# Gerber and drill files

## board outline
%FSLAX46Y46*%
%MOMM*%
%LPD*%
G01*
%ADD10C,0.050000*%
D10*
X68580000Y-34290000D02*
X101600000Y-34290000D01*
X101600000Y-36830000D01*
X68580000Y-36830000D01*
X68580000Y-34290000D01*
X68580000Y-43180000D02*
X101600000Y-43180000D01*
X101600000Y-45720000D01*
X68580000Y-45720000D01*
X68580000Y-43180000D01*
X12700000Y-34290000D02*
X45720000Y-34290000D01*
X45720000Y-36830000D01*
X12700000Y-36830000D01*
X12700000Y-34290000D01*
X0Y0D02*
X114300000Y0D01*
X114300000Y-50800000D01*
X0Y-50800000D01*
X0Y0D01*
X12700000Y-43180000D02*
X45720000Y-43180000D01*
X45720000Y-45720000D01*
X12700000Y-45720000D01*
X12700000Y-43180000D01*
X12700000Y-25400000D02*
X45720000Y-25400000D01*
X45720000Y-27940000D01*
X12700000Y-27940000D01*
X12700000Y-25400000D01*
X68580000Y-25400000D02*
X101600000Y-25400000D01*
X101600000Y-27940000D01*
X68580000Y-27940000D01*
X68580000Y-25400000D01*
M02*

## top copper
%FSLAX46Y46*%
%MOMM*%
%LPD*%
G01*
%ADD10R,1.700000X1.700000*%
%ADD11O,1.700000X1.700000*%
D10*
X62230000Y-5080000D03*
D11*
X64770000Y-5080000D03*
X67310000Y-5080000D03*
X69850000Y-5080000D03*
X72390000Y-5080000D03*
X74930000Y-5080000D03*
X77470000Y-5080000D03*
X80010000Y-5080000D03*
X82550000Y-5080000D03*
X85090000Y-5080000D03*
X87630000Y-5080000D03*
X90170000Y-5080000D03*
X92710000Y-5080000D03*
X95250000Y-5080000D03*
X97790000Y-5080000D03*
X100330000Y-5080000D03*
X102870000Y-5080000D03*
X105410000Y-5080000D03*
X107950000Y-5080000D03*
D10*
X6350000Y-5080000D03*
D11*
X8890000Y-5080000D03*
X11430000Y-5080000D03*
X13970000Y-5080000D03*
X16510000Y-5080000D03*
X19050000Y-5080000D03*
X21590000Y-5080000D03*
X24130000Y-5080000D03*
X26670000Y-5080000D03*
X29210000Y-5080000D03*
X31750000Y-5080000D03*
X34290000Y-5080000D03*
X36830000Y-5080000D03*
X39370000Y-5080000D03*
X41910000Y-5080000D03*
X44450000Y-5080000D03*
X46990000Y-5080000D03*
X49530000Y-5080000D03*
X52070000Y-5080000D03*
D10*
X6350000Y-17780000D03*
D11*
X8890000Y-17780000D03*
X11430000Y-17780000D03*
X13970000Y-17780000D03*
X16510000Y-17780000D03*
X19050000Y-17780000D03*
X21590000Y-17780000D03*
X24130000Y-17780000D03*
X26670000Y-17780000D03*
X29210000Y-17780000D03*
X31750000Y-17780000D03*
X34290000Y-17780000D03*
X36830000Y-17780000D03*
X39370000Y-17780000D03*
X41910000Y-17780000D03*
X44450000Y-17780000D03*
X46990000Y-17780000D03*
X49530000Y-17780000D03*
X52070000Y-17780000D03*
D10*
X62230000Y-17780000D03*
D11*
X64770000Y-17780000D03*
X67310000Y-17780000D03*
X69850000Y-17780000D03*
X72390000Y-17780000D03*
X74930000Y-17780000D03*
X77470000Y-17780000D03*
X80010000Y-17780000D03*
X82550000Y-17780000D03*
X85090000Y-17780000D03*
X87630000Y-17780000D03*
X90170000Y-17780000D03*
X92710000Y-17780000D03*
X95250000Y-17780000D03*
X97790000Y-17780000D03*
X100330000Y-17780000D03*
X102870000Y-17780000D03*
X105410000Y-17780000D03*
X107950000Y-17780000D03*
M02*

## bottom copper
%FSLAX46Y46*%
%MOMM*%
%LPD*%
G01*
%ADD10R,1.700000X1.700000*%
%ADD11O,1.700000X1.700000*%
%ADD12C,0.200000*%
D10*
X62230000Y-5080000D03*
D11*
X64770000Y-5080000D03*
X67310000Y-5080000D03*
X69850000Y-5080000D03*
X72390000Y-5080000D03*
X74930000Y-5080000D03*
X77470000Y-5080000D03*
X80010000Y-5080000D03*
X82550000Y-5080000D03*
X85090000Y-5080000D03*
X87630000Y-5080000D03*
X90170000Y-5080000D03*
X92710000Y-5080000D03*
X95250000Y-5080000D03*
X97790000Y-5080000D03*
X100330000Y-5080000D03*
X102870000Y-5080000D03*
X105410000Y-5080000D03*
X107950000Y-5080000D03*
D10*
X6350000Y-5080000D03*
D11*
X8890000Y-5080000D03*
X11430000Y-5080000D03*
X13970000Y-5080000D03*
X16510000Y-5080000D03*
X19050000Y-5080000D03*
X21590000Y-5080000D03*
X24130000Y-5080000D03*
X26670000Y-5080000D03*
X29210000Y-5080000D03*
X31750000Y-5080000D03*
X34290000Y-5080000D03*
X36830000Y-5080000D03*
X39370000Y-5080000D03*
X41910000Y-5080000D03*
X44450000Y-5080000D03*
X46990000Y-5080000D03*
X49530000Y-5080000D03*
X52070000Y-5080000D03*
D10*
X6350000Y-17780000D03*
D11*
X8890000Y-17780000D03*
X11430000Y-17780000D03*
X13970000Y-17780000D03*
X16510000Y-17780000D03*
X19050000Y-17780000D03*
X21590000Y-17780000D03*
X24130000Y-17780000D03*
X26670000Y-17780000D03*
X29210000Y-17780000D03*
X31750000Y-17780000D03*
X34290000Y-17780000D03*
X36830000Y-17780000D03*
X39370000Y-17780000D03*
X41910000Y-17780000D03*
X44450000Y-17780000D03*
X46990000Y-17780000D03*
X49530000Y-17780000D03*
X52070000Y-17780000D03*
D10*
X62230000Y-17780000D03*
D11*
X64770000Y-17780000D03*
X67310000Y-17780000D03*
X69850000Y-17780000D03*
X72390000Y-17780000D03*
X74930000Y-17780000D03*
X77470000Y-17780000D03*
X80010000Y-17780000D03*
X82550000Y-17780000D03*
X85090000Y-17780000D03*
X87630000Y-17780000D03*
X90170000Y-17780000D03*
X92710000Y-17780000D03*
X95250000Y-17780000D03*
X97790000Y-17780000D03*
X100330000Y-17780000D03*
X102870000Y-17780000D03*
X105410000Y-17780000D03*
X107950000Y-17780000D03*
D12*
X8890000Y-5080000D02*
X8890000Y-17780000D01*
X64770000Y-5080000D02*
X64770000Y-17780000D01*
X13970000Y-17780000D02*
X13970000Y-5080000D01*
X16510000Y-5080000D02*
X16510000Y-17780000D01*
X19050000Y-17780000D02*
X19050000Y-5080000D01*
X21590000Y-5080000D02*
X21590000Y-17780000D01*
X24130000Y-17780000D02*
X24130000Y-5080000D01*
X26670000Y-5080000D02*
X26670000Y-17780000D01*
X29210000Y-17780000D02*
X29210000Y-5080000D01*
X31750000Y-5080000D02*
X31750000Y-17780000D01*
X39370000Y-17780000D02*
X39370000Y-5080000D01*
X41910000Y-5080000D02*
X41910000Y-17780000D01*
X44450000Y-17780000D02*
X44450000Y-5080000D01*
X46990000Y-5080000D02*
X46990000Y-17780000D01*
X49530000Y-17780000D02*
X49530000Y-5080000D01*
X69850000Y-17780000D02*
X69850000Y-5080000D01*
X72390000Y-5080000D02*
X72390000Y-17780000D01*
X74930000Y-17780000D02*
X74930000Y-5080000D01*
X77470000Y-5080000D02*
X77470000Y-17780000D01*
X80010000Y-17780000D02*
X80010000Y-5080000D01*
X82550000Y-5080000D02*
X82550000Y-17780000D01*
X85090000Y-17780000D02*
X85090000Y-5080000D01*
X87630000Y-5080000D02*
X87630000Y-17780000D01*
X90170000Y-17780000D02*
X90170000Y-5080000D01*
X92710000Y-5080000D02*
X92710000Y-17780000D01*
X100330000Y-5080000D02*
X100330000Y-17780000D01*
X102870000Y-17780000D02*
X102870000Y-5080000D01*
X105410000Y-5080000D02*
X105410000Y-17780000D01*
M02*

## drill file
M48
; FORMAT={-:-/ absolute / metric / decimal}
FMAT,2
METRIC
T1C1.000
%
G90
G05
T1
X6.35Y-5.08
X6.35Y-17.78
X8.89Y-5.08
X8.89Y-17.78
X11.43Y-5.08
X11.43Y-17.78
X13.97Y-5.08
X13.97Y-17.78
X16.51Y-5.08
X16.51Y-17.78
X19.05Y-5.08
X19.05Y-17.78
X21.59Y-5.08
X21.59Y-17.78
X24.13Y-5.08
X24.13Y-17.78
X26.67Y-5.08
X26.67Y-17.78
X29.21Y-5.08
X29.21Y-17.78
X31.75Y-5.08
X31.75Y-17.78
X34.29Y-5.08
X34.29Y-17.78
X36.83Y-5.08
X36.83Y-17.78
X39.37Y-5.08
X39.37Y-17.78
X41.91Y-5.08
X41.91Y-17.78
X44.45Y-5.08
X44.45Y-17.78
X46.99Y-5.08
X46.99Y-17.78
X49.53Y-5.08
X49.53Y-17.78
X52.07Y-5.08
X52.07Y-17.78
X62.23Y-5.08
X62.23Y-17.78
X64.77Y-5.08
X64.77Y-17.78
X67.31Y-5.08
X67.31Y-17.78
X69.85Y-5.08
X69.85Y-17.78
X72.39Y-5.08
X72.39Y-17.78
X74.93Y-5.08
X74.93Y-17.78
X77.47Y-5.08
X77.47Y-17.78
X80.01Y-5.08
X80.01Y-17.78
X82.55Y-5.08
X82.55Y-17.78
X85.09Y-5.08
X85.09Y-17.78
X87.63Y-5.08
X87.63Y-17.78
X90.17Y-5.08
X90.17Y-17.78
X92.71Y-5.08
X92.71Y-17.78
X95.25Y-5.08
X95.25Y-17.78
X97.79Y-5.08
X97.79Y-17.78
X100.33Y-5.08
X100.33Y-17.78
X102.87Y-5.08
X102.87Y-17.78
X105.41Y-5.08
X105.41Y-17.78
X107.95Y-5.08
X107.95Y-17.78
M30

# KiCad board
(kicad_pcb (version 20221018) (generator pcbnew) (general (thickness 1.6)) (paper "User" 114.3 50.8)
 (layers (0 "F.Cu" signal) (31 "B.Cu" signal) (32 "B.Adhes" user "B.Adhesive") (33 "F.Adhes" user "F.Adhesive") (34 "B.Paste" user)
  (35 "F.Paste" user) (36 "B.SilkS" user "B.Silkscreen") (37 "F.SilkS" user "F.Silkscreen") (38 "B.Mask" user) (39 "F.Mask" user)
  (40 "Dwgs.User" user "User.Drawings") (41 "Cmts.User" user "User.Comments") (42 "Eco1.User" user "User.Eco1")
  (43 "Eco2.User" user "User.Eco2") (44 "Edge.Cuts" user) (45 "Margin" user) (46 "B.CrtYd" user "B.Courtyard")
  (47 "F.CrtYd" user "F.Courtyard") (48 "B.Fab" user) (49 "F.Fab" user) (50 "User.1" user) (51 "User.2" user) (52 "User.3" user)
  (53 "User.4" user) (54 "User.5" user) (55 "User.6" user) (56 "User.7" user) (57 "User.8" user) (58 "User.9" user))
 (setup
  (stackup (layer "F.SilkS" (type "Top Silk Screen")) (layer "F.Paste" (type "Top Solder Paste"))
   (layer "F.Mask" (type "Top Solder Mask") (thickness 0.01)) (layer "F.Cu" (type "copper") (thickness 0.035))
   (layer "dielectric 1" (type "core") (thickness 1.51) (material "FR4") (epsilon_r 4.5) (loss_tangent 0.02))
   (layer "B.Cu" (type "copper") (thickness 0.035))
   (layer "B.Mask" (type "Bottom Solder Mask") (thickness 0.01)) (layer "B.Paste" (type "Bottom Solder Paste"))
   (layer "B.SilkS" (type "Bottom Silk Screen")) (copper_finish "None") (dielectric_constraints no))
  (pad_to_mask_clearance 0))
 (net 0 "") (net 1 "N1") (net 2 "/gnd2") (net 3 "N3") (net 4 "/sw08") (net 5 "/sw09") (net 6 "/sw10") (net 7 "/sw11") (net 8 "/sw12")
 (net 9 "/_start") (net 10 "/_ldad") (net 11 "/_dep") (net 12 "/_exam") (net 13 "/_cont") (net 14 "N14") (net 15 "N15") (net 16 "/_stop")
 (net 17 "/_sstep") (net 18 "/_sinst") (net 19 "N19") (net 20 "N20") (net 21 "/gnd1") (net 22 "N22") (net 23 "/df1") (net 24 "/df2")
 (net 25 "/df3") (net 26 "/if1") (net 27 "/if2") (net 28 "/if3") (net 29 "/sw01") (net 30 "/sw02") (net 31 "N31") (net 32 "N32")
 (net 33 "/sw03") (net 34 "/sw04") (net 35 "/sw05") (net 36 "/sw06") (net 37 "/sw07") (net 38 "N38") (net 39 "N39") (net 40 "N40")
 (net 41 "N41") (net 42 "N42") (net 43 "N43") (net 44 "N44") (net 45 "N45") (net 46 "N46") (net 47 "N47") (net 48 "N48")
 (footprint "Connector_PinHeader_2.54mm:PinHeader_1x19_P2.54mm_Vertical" (layer "F.Cu") (at 62.23 5.08 90)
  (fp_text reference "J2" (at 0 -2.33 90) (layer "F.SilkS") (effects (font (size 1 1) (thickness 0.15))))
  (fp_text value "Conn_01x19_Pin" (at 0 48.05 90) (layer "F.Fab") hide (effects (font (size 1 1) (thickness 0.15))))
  (pad "1" thru_hole rect (at 0 0 90) (size 1.7 1.7) (drill 1) (layers "*.Cu" "*.Mask") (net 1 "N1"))
  (pad "2" thru_hole oval (at 0 2.54 90) (size 1.7 1.7) (drill 1) (layers "*.Cu" "*.Mask") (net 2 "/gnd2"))
  (pad "3" thru_hole oval (at 0 5.08 90) (size 1.7 1.7) (drill 1) (layers "*.Cu" "*.Mask") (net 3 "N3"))
  (pad "4" thru_hole oval (at 0 7.62 90) (size 1.7 1.7) (drill 1) (layers "*.Cu" "*.Mask") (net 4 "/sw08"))
  (pad "5" thru_hole oval (at 0 10.16 90) (size 1.7 1.7) (drill 1) (layers "*.Cu" "*.Mask") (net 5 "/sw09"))
  (pad "6" thru_hole oval (at 0 12.7 90) (size 1.7 1.7) (drill 1) (layers "*.Cu" "*.Mask") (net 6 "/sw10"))
  (pad "7" thru_hole oval (at 0 15.24 90) (size 1.7 1.7) (drill 1) (layers "*.Cu" "*.Mask") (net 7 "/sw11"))
  (pad "8" thru_hole oval (at 0 17.78 90) (size 1.7 1.7) (drill 1) (layers "*.Cu" "*.Mask") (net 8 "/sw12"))
  (pad "9" thru_hole oval (at 0 20.32 90) (size 1.7 1.7) (drill 1) (layers "*.Cu" "*.Mask") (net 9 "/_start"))
  (pad "10" thru_hole oval (at 0 22.86 90) (size 1.7 1.7) (drill 1) (layers "*.Cu" "*.Mask") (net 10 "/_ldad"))
  (pad "11" thru_hole oval (at 0 25.4 90) (size 1.7 1.7) (drill 1) (layers "*.Cu" "*.Mask") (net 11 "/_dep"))
  (pad "12" thru_hole oval (at 0 27.94 90) (size 1.7 1.7) (drill 1) (layers "*.Cu" "*.Mask") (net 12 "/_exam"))
  (pad "13" thru_hole oval (at 0 30.48 90) (size 1.7 1.7) (drill 1) (layers "*.Cu" "*.Mask") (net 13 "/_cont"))
  (pad "14" thru_hole oval (at 0 33.02 90) (size 1.7 1.7) (drill 1) (layers "*.Cu" "*.Mask") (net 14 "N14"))
  (pad "15" thru_hole oval (at 0 35.56 90) (size 1.7 1.7) (drill 1) (layers "*.Cu" "*.Mask") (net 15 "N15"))
  (pad "16" thru_hole oval (at 0 38.1 90) (size 1.7 1.7) (drill 1) (layers "*.Cu" "*.Mask") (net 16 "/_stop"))
  (pad "17" thru_hole oval (at 0 40.64 90) (size 1.7 1.7) (drill 1) (layers "*.Cu" "*.Mask") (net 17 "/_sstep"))
  (pad "18" thru_hole oval (at 0 43.18 90) (size 1.7 1.7) (drill 1) (layers "*.Cu" "*.Mask") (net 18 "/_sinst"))
  (pad "19" thru_hole oval (at 0 45.72 90) (size 1.7 1.7) (drill 1) (layers "*.Cu" "*.Mask") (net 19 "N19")))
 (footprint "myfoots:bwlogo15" (layer "F.Cu") (at 312.42 12.7)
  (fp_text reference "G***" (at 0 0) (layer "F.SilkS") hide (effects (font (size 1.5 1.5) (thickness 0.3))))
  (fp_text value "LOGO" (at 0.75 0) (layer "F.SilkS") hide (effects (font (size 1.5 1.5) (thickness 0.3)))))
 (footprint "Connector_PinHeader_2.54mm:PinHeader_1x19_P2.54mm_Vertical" (layer "F.Cu") (at 6.35 5.08 90)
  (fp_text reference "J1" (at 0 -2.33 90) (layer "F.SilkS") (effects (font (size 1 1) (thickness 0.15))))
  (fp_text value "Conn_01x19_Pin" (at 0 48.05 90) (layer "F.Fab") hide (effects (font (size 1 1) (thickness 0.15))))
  (pad "1" thru_hole rect (at 0 0 90) (size 1.7 1.7) (drill 1) (layers "*.Cu" "*.Mask") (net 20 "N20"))
  (pad "2" thru_hole oval (at 0 2.54 90) (size 1.7 1.7) (drill 1) (layers "*.Cu" "*.Mask") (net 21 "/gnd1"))
  (pad "3" thru_hole oval (at 0 5.08 90) (size 1.7 1.7) (drill 1) (layers "*.Cu" "*.Mask") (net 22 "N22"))
  (pad "4" thru_hole oval (at 0 7.62 90) (size 1.7 1.7) (drill 1) (layers "*.Cu" "*.Mask") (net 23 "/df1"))
  (pad "5" thru_hole oval (at 0 10.16 90) (size 1.7 1.7) (drill 1) (layers "*.Cu" "*.Mask") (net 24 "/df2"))
  (pad "6" thru_hole oval (at 0 12.7 90) (size 1.7 1.7) (drill 1) (layers "*.Cu" "*.Mask") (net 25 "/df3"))
  (pad "7" thru_hole oval (at 0 15.24 90) (size 1.7 1.7) (drill 1) (layers "*.Cu" "*.Mask") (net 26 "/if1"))
  (pad "8" thru_hole oval (at 0 17.78 90) (size 1.7 1.7) (drill 1) (layers "*.Cu" "*.Mask") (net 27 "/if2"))
  (pad "9" thru_hole oval (at 0 20.32 90) (size 1.7 1.7) (drill 1) (layers "*.Cu" "*.Mask") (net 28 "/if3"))
  (pad "10" thru_hole oval (at 0 22.86 90) (size 1.7 1.7) (drill 1) (layers "*.Cu" "*.Mask") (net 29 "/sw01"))
  (pad "11" thru_hole oval (at 0 25.4 90) (size 1.7 1.7) (drill 1) (layers "*.Cu" "*.Mask") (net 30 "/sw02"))
  (pad "12" thru_hole oval (at 0 27.94 90) (size 1.7 1.7) (drill 1) (layers "*.Cu" "*.Mask") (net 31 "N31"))
  (pad "13" thru_hole oval (at 0 30.48 90) (size 1.7 1.7) (drill 1) (layers "*.Cu" "*.Mask") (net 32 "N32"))
  (pad "14" thru_hole oval (at 0 33.02 90) (size 1.7 1.7) (drill 1) (layers "*.Cu" "*.Mask") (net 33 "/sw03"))
  (pad "15" thru_hole oval (at 0 35.56 90) (size 1.7 1.7) (drill 1) (layers "*.Cu" "*.Mask") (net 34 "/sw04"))
  (pad "16" thru_hole oval (at 0 38.1 90) (size 1.7 1.7) (drill 1) (layers "*.Cu" "*.Mask") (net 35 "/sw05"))
  (pad "17" thru_hole oval (at 0 40.64 90) (size 1.7 1.7) (drill 1) (layers "*.Cu" "*.Mask") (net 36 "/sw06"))
  (pad "18" thru_hole oval (at 0 43.18 90) (size 1.7 1.7) (drill 1) (layers "*.Cu" "*.Mask") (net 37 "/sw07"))
  (pad "19" thru_hole oval (at 0 45.72 90) (size 1.7 1.7) (drill 1) (layers "*.Cu" "*.Mask") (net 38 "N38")))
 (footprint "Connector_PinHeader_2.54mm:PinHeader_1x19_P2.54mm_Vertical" (layer "F.Cu") (at 6.35 17.78 90)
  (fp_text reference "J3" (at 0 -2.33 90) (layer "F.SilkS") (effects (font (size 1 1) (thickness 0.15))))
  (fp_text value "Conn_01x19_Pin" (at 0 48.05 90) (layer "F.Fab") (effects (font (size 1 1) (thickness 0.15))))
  (pad "1" thru_hole rect (at 0 0 90) (size 1.7 1.7) (drill 1) (layers "*.Cu" "*.Mask") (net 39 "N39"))
  (pad "2" thru_hole oval (at 0 2.54 90) (size 1.7 1.7) (drill 1) (layers "*.Cu" "*.Mask") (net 21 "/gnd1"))
  (pad "3" thru_hole oval (at 0 5.08 90) (size 1.7 1.7) (drill 1) (layers "*.Cu" "*.Mask") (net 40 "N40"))
  (pad "4" thru_hole oval (at 0 7.62 90) (size 1.7 1.7) (drill 1) (layers "*.Cu" "*.Mask") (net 23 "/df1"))
  (pad "5" thru_hole oval (at 0 10.16 90) (size 1.7 1.7) (drill 1) (layers "*.Cu" "*.Mask") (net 24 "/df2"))
  (pad "6" thru_hole oval (at 0 12.7 90) (size 1.7 1.7) (drill 1) (layers "*.Cu" "*.Mask") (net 25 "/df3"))
  (pad "7" thru_hole oval (at 0 15.24 90) (size 1.7 1.7) (drill 1) (layers "*.Cu" "*.Mask") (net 26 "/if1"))
  (pad "8" thru_hole oval (at 0 17.78 90) (size 1.7 1.7) (drill 1) (layers "*.Cu" "*.Mask") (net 27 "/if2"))
  (pad "9" thru_hole oval (at 0 20.32 90) (size 1.7 1.7) (drill 1) (layers "*.Cu" "*.Mask") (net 28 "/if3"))
  (pad "10" thru_hole oval (at 0 22.86 90) (size 1.7 1.7) (drill 1) (layers "*.Cu" "*.Mask") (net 29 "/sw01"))
  (pad "11" thru_hole oval (at 0 25.4 90) (size 1.7 1.7) (drill 1) (layers "*.Cu" "*.Mask") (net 30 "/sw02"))
  (pad "12" thru_hole oval (at 0 27.94 90) (size 1.7 1.7) (drill 1) (layers "*.Cu" "*.Mask") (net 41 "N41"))
  (pad "13" thru_hole oval (at 0 30.48 90) (size 1.7 1.7) (drill 1) (layers "*.Cu" "*.Mask") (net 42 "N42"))
  (pad "14" thru_hole oval (at 0 33.02 90) (size 1.7 1.7) (drill 1) (layers "*.Cu" "*.Mask") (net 33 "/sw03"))
  (pad "15" thru_hole oval (at 0 35.56 90) (size 1.7 1.7) (drill 1) (layers "*.Cu" "*.Mask") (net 34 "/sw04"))
  (pad "16" thru_hole oval (at 0 38.1 90) (size 1.7 1.7) (drill 1) (layers "*.Cu" "*.Mask") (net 35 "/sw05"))
  (pad "17" thru_hole oval (at 0 40.64 90) (size 1.7 1.7) (drill 1) (layers "*.Cu" "*.Mask") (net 36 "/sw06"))
  (pad "18" thru_hole oval (at 0 43.18 90) (size 1.7 1.7) (drill 1) (layers "*.Cu" "*.Mask") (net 37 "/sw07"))
  (pad "19" thru_hole oval (at 0 45.72 90) (size 1.7 1.7) (drill 1) (layers "*.Cu" "*.Mask") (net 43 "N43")))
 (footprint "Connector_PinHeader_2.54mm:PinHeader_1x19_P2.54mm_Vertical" (layer "F.Cu") (at 62.23 17.78 90)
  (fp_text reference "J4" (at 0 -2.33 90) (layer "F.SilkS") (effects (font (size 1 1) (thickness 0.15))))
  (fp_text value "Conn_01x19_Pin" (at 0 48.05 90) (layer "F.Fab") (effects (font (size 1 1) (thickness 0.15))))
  (pad "1" thru_hole rect (at 0 0 90) (size 1.7 1.7) (drill 1) (layers "*.Cu" "*.Mask") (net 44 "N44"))
  (pad "2" thru_hole oval (at 0 2.54 90) (size 1.7 1.7) (drill 1) (layers "*.Cu" "*.Mask") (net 2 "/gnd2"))
  (pad "3" thru_hole oval (at 0 5.08 90) (size 1.7 1.7) (drill 1) (layers "*.Cu" "*.Mask") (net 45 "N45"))
  (pad "4" thru_hole oval (at 0 7.62 90) (size 1.7 1.7) (drill 1) (layers "*.Cu" "*.Mask") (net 4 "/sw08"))
  (pad "5" thru_hole oval (at 0 10.16 90) (size 1.7 1.7) (drill 1) (layers "*.Cu" "*.Mask") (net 5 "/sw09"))
  (pad "6" thru_hole oval (at 0 12.7 90) (size 1.7 1.7) (drill 1) (layers "*.Cu" "*.Mask") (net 6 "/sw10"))
  (pad "7" thru_hole oval (at 0 15.24 90) (size 1.7 1.7) (drill 1) (layers "*.Cu" "*.Mask") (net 7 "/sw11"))
  (pad "8" thru_hole oval (at 0 17.78 90) (size 1.7 1.7) (drill 1) (layers "*.Cu" "*.Mask") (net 8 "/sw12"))
  (pad "9" thru_hole oval (at 0 20.32 90) (size 1.7 1.7) (drill 1) (layers "*.Cu" "*.Mask") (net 9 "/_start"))
  (pad "10" thru_hole oval (at 0 22.86 90) (size 1.7 1.7) (drill 1) (layers "*.Cu" "*.Mask") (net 10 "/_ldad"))
  (pad "11" thru_hole oval (at 0 25.4 90) (size 1.7 1.7) (drill 1) (layers "*.Cu" "*.Mask") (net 11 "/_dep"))
  (pad "12" thru_hole oval (at 0 27.94 90) (size 1.7 1.7) (drill 1) (layers "*.Cu" "*.Mask") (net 12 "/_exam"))
  (pad "13" thru_hole oval (at 0 30.48 90) (size 1.7 1.7) (drill 1) (layers "*.Cu" "*.Mask") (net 13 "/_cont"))
  (pad "14" thru_hole oval (at 0 33.02 90) (size 1.7 1.7) (drill 1) (layers "*.Cu" "*.Mask") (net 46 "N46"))
  (pad "15" thru_hole oval (at 0 35.56 90) (size 1.7 1.7) (drill 1) (layers "*.Cu" "*.Mask") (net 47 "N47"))
  (pad "16" thru_hole oval (at 0 38.1 90) (size 1.7 1.7) (drill 1) (layers "*.Cu" "*.Mask") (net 16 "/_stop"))
  (pad "17" thru_hole oval (at 0 40.64 90) (size 1.7 1.7) (drill 1) (layers "*.Cu" "*.Mask") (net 17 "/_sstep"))
  (pad "18" thru_hole oval (at 0 43.18 90) (size 1.7 1.7) (drill 1) (layers "*.Cu" "*.Mask") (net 18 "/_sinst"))
  (pad "19" thru_hole oval (at 0 45.72 90) (size 1.7 1.7) (drill 1) (layers "*.Cu" "*.Mask") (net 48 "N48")))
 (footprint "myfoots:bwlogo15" (layer "B.Cu") (at 341.63 12.7 180)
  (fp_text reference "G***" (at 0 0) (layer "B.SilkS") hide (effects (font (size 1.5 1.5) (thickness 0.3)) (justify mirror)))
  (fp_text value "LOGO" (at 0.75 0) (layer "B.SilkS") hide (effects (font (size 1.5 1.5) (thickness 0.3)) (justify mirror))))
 (gr_rect (start 68.58 34.29) (end 101.6 36.83) (stroke (width 0.05) (type default)) (fill none) (layer "Edge.Cuts"))
 (gr_rect (start 68.58 43.18) (end 101.6 45.72) (stroke (width 0.05) (type default)) (fill none) (layer "Edge.Cuts"))
 (gr_rect (start 12.7 34.29) (end 45.72 36.83) (stroke (width 0.05) (type default)) (fill none) (layer "Edge.Cuts"))
 (gr_rect (start 0 0) (end 114.3 50.8) (stroke (width 0.05) (type default)) (fill none) (layer "Edge.Cuts"))
 (gr_rect (start 12.7 43.18) (end 45.72 45.72) (stroke (width 0.05) (type default)) (fill none) (layer "Edge.Cuts"))
 (gr_rect (start 12.7 25.4) (end 45.72 27.94) (stroke (width 0.05) (type default)) (fill none) (layer "Edge.Cuts"))
 (gr_rect (start 68.58 25.4) (end 101.6 27.94) (stroke (width 0.05) (type default)) (fill none) (layer "Edge.Cuts"))
 (segment (start 8.89 5.08) (end 8.89 17.78) (width 0.2) (layer "B.Cu") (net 21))
 (segment (start 64.77 5.08) (end 64.77 17.78) (width 0.2) (layer "B.Cu") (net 2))
 (segment (start 13.97 17.78) (end 13.97 5.08) (width 0.2) (layer "B.Cu") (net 23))
 (segment (start 16.51 5.08) (end 16.51 17.78) (width 0.2) (layer "B.Cu") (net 24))
 (segment (start 19.05 17.78) (end 19.05 5.08) (width 0.2) (layer "B.Cu") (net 25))
 (segment (start 21.59 5.08) (end 21.59 17.78) (width 0.2) (layer "B.Cu") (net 26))
 (segment (start 24.13 17.78) (end 24.13 5.08) (width 0.2) (layer "B.Cu") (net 27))
 (segment (start 26.67 5.08) (end 26.67 17.78) (width 0.2) (layer "B.Cu") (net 28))
 (segment (start 29.21 17.78) (end 29.21 5.08) (width 0.2) (layer "B.Cu") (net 29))
 (segment (start 31.75 5.08) (end 31.75 17.78) (width 0.2) (layer "B.Cu") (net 30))
 (segment (start 39.37 17.78) (end 39.37 5.08) (width 0.2) (layer "B.Cu") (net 33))
 (segment (start 41.91 5.08) (end 41.91 17.78) (width 0.2) (layer "B.Cu") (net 34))
 (segment (start 44.45 17.78) (end 44.45 5.08) (width 0.2) (layer "B.Cu") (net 35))
 (segment (start 46.99 5.08) (end 46.99 17.78) (width 0.2) (layer "B.Cu") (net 36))
 (segment (start 49.53 17.78) (end 49.53 5.08) (width 0.2) (layer "B.Cu") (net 37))
 (segment (start 69.85 17.78) (end 69.85 5.08) (width 0.2) (layer "B.Cu") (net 4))
 (segment (start 72.39 5.08) (end 72.39 17.78) (width 0.2) (layer "B.Cu") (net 5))
 (segment (start 74.93 17.78) (end 74.93 5.08) (width 0.2) (layer "B.Cu") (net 6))
 (segment (start 77.47 5.08) (end 77.47 17.78) (width 0.2) (layer "B.Cu") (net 7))
 (segment (start 80.01 17.78) (end 80.01 5.08) (width 0.2) (layer "B.Cu") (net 8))
 (segment (start 82.55 5.08) (end 82.55 17.78) (width 0.2) (layer "B.Cu") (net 9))
 (segment (start 85.09 17.78) (end 85.09 5.08) (width 0.2) (layer "B.Cu") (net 10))
 (segment (start 87.63 5.08) (end 87.63 17.78) (width 0.2) (layer "B.Cu") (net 11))
 (segment (start 90.17 17.78) (end 90.17 5.08) (width 0.2) (layer "B.Cu") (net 12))
 (segment (start 92.71 5.08) (end 92.71 17.78) (width 0.2) (layer "B.Cu") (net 13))
 (segment (start 100.33 5.08) (end 100.33 17.78) (width 0.2) (layer "B.Cu") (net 16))
 (segment (start 102.87 17.78) (end 102.87 5.08) (width 0.2) (layer "B.Cu") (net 17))
 (segment (start 105.41 5.08) (end 105.41 17.78) (width 0.2) (layer "B.Cu") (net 18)))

